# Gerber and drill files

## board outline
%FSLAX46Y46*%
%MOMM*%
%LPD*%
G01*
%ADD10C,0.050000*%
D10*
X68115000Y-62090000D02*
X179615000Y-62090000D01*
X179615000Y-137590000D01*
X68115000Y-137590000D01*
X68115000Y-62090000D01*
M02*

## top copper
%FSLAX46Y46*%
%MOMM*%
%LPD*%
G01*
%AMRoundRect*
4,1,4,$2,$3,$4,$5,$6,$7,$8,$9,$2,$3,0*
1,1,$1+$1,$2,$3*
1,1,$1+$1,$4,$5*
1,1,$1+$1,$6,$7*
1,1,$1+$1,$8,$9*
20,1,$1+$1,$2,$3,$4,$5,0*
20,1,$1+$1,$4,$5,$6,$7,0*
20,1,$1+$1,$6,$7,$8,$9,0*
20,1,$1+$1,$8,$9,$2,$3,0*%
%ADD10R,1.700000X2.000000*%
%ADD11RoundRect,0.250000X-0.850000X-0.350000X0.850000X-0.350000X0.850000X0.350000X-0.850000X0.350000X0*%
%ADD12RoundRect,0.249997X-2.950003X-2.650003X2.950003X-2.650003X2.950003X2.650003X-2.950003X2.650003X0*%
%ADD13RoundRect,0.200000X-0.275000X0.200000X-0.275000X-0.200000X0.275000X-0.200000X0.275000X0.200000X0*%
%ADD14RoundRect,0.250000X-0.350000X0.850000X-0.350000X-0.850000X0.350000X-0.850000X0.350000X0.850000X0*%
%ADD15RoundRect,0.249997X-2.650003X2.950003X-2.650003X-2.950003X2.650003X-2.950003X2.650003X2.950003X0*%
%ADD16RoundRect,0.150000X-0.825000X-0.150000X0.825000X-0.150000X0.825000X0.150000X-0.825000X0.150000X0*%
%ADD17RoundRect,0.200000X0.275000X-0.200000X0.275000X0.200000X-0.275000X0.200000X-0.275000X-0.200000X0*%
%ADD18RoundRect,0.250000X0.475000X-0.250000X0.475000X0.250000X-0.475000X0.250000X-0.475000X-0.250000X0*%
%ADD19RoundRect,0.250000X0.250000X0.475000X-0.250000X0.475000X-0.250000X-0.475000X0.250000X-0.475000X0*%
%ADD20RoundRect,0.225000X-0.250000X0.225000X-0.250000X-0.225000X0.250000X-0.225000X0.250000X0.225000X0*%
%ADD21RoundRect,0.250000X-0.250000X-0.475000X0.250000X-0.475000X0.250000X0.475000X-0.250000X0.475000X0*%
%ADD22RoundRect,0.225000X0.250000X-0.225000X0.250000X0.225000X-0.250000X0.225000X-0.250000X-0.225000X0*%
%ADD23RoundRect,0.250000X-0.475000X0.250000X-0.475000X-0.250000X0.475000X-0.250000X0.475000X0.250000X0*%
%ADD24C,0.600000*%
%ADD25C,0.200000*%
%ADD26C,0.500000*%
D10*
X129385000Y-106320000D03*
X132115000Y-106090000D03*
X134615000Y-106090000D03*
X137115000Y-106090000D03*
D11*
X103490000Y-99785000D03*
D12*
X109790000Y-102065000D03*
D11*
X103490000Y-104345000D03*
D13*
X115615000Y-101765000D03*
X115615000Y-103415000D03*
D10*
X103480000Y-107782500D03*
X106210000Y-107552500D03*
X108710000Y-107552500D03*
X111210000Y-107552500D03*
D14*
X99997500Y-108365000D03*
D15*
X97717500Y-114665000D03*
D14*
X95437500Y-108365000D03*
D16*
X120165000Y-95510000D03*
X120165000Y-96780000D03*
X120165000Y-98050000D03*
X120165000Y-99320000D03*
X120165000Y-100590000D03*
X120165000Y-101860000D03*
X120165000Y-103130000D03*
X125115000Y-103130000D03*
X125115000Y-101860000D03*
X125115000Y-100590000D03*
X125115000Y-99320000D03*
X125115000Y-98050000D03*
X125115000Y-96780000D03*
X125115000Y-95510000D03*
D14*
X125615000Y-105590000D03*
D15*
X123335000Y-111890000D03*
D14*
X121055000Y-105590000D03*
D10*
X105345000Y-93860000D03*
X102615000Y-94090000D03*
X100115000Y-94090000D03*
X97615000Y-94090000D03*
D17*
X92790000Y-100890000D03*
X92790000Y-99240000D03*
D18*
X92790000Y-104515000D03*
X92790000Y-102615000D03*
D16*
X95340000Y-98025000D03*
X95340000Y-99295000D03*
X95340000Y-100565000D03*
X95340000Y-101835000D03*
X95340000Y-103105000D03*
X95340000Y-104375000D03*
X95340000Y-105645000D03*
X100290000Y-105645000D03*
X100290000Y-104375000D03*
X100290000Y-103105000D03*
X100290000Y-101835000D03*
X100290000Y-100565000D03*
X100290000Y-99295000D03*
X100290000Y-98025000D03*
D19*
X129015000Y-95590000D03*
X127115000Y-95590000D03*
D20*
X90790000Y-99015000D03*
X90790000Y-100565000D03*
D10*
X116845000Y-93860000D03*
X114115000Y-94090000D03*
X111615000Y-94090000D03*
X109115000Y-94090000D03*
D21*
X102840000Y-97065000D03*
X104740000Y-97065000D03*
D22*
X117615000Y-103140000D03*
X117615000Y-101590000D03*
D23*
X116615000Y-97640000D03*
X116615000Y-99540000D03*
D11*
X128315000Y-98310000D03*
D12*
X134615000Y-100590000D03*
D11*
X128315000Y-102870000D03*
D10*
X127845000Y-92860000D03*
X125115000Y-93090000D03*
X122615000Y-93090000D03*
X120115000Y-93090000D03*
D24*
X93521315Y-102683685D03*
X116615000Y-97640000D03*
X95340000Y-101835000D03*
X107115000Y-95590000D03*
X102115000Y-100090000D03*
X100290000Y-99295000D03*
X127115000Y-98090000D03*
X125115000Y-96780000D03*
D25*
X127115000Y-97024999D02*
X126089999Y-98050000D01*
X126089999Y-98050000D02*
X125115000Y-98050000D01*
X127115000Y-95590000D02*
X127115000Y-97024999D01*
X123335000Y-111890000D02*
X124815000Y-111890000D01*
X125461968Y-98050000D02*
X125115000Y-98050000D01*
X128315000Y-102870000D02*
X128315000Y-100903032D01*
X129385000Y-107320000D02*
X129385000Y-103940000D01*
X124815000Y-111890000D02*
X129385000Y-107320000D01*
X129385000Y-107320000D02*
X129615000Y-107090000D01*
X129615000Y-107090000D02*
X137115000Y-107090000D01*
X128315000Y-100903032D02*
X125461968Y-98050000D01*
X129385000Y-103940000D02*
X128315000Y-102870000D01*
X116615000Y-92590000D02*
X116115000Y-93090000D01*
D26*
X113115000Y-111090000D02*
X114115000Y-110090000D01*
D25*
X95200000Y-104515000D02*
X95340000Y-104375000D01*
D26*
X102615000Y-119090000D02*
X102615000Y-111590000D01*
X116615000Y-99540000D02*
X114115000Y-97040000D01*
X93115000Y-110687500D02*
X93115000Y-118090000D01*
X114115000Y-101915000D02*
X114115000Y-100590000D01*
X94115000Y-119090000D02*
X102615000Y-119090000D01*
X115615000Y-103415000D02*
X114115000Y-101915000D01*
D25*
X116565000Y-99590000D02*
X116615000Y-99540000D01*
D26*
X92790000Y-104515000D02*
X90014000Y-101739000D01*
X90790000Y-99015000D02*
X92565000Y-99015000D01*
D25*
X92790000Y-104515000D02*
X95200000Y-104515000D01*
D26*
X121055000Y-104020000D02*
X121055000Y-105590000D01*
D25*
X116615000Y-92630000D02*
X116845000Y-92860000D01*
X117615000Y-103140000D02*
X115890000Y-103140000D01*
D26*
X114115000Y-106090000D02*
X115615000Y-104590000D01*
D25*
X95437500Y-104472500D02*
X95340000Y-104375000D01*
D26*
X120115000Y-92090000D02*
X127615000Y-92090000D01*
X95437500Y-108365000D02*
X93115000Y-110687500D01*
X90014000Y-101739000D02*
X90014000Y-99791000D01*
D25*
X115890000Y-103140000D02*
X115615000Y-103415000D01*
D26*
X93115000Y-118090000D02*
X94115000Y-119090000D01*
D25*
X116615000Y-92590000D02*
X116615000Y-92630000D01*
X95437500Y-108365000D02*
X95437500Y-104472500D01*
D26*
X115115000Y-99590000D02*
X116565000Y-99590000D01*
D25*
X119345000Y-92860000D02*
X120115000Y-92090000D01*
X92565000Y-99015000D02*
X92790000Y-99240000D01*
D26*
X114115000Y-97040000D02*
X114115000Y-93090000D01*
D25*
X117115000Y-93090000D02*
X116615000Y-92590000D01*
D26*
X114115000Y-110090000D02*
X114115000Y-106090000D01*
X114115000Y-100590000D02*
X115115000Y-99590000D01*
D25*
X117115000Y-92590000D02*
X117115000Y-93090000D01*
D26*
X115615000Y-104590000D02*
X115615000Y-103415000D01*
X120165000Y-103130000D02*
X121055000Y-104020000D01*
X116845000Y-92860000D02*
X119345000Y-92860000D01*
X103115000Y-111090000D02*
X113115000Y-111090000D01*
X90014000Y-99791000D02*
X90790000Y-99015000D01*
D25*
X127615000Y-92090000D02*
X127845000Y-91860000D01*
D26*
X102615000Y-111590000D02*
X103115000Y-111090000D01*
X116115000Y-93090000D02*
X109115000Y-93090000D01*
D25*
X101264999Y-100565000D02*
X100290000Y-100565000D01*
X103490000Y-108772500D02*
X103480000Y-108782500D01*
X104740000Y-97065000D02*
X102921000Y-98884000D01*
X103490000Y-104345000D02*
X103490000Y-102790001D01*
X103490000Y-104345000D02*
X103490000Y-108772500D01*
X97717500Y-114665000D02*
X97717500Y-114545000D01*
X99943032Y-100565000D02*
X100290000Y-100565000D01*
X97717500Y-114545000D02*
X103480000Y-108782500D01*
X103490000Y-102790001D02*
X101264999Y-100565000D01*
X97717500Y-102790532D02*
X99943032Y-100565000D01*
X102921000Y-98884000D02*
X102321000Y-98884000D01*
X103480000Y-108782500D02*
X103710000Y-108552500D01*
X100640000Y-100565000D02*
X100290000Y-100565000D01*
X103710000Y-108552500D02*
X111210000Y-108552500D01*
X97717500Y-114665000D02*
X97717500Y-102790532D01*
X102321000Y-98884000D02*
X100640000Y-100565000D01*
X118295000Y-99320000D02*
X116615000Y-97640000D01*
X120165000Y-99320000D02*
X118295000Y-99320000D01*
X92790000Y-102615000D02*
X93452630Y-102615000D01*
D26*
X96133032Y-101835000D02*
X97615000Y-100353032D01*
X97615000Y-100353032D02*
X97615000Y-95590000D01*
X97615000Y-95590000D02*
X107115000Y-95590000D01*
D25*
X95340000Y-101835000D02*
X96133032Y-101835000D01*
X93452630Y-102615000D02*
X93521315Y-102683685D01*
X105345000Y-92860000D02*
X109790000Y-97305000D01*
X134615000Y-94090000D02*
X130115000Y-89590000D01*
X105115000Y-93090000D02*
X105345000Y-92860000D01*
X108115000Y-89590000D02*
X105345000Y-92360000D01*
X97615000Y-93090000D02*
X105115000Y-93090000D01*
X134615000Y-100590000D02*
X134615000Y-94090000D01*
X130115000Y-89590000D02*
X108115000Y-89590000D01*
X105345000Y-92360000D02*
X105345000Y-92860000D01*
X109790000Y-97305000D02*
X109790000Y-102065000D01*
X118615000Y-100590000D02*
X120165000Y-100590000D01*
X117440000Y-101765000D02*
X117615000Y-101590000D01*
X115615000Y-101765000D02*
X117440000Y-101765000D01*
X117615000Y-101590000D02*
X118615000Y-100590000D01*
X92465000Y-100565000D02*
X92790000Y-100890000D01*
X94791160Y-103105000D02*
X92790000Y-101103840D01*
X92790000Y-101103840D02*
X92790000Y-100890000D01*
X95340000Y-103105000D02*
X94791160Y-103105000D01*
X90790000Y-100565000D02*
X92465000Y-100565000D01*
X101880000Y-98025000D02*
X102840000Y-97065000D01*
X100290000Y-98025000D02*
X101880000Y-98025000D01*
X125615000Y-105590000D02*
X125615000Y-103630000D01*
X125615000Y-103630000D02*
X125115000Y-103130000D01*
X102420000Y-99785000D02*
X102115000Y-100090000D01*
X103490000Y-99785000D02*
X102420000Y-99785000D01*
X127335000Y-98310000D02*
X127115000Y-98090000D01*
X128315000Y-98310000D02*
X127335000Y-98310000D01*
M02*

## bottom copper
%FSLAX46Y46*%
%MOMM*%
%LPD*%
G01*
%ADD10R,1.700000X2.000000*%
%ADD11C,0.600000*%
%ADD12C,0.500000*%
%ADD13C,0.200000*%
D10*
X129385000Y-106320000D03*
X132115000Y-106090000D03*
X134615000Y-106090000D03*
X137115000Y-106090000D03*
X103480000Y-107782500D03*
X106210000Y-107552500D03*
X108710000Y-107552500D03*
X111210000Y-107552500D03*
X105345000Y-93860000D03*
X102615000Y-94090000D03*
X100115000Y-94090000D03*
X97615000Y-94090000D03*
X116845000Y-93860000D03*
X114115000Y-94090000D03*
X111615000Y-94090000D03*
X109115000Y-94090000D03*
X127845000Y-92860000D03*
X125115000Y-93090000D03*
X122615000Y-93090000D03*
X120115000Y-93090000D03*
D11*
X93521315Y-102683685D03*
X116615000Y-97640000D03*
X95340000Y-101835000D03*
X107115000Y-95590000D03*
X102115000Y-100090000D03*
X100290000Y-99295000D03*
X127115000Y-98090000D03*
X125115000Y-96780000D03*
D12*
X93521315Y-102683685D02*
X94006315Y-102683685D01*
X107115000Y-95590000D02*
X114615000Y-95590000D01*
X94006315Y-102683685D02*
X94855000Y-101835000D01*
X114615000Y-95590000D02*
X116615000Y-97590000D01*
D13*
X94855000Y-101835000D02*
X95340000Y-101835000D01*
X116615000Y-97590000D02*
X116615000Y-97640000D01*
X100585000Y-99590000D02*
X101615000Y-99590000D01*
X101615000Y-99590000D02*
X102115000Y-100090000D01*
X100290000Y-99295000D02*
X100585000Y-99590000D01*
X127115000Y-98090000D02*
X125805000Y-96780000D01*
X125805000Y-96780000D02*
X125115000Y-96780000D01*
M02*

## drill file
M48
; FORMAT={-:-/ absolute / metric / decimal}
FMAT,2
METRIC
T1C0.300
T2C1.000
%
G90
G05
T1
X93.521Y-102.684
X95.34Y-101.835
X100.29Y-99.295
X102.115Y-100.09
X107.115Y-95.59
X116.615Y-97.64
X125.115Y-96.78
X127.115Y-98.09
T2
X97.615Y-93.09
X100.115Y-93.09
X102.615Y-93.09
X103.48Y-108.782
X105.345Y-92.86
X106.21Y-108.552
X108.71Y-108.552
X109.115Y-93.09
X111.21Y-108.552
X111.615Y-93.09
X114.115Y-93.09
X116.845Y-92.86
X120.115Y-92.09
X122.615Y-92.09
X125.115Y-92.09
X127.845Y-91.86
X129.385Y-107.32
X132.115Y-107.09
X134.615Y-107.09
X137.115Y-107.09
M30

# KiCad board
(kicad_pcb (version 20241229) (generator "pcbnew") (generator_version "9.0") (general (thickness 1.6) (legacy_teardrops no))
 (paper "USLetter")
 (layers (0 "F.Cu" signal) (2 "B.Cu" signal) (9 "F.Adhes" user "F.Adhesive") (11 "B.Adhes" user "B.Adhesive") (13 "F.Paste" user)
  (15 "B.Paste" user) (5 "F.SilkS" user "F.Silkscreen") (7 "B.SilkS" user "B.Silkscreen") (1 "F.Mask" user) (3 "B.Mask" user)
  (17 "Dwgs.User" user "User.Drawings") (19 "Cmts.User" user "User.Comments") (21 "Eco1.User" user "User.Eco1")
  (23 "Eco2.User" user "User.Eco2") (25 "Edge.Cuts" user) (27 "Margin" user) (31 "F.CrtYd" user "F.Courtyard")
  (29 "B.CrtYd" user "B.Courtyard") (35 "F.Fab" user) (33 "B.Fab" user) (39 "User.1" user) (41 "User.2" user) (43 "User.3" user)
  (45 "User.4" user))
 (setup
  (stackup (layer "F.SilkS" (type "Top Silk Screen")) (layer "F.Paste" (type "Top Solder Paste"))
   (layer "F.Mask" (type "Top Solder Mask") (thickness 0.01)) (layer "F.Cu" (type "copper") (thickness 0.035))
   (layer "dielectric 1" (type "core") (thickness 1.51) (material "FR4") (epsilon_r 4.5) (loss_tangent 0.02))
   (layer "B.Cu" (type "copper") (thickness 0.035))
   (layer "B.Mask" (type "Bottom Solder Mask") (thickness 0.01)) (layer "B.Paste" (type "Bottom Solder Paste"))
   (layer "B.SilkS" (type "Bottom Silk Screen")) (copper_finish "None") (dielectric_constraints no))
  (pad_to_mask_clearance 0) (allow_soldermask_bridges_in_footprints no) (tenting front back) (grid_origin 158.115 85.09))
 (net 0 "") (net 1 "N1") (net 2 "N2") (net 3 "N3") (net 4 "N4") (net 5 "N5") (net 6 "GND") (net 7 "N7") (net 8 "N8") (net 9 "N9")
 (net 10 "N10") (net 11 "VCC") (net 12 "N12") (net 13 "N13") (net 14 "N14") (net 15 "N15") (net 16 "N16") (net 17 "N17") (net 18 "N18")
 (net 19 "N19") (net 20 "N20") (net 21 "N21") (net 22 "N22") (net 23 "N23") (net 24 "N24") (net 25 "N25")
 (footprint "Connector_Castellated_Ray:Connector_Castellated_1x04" (layer "F.Cu") (at 132.115 106.09 90)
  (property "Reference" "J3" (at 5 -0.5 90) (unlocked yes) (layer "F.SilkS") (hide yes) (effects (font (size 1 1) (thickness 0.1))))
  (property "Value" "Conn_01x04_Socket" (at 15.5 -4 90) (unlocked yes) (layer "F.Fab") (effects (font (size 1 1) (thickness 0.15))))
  (pad "1" thru_hole rect (at -1.23 -2.73 90) (size 2 1.7) (drill 1 (offset 1 0)) (layers "*.Cu" "*.Mask") (remove_unused_layers no)
   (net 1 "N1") (solder_mask_margin 0.04))
  (pad "2" thru_hole rect (at -1 0 90) (size 2 1.7) (drill 1 (offset 1 0)) (layers "*.Cu" "*.Mask") (remove_unused_layers no) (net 1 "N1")
   (solder_mask_margin 0.04))
  (pad "3" thru_hole rect (at -1 2.5 90) (size 2 1.7) (drill 1 (offset 1 0)) (layers "*.Cu" "*.Mask") (remove_unused_layers no) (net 1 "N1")
   (solder_mask_margin 0.04))
  (pad "4" thru_hole rect (at -1 5 90) (size 2 1.7) (drill 1 (offset 1 0)) (layers "*.Cu" "*.Mask") (remove_unused_layers no) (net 1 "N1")
   (solder_mask_margin 0.04)))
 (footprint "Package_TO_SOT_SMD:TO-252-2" (layer "F.Cu") (at 108.53 102.065)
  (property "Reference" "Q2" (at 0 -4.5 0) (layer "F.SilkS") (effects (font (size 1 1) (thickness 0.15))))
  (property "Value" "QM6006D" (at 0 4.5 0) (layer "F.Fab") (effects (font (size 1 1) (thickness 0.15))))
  (pad "" smd roundrect (at -0.415 -1.525) (size 3.05 2.75) (layers "F.Paste") (roundrect_rratio 0.090909))
  (pad "" smd roundrect (at -0.415 1.525) (size 3.05 2.75) (layers "F.Paste") (roundrect_rratio 0.090909))
  (pad "" smd roundrect (at 2.935 -1.525) (size 3.05 2.75) (layers "F.Paste") (roundrect_rratio 0.090909))
  (pad "" smd roundrect (at 2.935 1.525) (size 3.05 2.75) (layers "F.Paste") (roundrect_rratio 0.090909))
  (pad "1" smd roundrect (at -5.04 -2.28) (size 2.2 1.2) (layers "F.Cu" "F.Mask" "F.Paste") (roundrect_rratio 0.208333) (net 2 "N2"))
  (pad "2" smd roundrect (at 1.26 0) (size 6.4 5.8) (layers "F.Cu" "F.Mask") (roundrect_rratio 0.043103) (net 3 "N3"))
  (pad "3" smd roundrect (at -5.04 2.28) (size 2.2 1.2) (layers "F.Cu" "F.Mask" "F.Paste") (roundrect_rratio 0.208333) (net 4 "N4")))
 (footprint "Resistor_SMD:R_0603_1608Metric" (layer "F.Cu") (at 115.615 102.59 -90)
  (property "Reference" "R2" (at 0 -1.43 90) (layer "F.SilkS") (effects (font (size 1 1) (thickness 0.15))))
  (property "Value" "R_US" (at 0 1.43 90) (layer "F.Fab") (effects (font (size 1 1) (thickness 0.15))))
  (pad "1" smd roundrect (at -0.825 0 270) (size 0.8 0.95) (layers "F.Cu" "F.Mask" "F.Paste") (roundrect_rratio 0.25) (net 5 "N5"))
  (pad "2" smd roundrect (at 0.825 0 270) (size 0.8 0.95) (layers "F.Cu" "F.Mask" "F.Paste") (roundrect_rratio 0.25) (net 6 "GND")))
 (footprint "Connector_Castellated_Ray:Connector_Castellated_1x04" (layer "F.Cu") (at 106.21 107.5525 90)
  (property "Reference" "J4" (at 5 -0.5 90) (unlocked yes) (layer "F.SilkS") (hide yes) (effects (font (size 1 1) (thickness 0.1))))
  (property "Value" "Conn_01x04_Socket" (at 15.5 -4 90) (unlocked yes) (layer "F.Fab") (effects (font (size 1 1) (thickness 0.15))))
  (pad "1" thru_hole rect (at -1.23 -2.73 90) (size 2 1.7) (drill 1 (offset 1 0)) (layers "*.Cu" "*.Mask") (remove_unused_layers no)
   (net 4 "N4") (solder_mask_margin 0.04))
  (pad "2" thru_hole rect (at -1 0 90) (size 2 1.7) (drill 1 (offset 1 0)) (layers "*.Cu" "*.Mask") (remove_unused_layers no) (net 4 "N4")
   (solder_mask_margin 0.04))
  (pad "3" thru_hole rect (at -1 2.5 90) (size 2 1.7) (drill 1 (offset 1 0)) (layers "*.Cu" "*.Mask") (remove_unused_layers no) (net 4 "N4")
   (solder_mask_margin 0.04))
  (pad "4" thru_hole rect (at -1 5 90) (size 2 1.7) (drill 1 (offset 1 0)) (layers "*.Cu" "*.Mask") (remove_unused_layers no) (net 4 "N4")
   (solder_mask_margin 0.04)))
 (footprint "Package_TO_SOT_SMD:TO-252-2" (layer "F.Cu") (at 97.7175 113.405 -90)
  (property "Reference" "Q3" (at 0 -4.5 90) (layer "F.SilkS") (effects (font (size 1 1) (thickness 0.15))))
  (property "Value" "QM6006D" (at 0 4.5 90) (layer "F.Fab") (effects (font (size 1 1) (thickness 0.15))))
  (pad "" smd roundrect (at -0.415 -1.525 270) (size 3.05 2.75) (layers "F.Paste") (roundrect_rratio 0.090909))
  (pad "" smd roundrect (at -0.415 1.525 270) (size 3.05 2.75) (layers "F.Paste") (roundrect_rratio 0.090909))
  (pad "" smd roundrect (at 2.935 -1.525 270) (size 3.05 2.75) (layers "F.Paste") (roundrect_rratio 0.090909))
  (pad "" smd roundrect (at 2.935 1.525 270) (size 3.05 2.75) (layers "F.Paste") (roundrect_rratio 0.090909))
  (pad "1" smd roundrect (at -5.04 -2.28 270) (size 2.2 1.2) (layers "F.Cu" "F.Mask" "F.Paste") (roundrect_rratio 0.208333) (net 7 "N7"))
  (pad "2" smd roundrect (at 1.26 0 270) (size 6.4 5.8) (layers "F.Cu" "F.Mask") (roundrect_rratio 0.043103) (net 4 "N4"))
  (pad "3" smd roundrect (at -5.04 2.28 270) (size 2.2 1.2) (layers "F.Cu" "F.Mask" "F.Paste") (roundrect_rratio 0.208333) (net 6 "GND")))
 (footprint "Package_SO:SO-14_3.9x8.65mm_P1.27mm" (layer "F.Cu") (at 122.64 99.32)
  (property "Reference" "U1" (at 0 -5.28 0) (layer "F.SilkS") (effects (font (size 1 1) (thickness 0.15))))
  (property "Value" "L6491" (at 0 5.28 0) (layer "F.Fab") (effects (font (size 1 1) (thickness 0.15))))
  (pad "1" smd roundrect (at -2.475 -3.81) (size 1.95 0.6) (layers "F.Cu" "F.Mask" "F.Paste") (roundrect_rratio 0.25) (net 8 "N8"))
  (pad "2" smd roundrect (at -2.475 -2.54) (size 1.95 0.6) (layers "F.Cu" "F.Mask" "F.Paste") (roundrect_rratio 0.25) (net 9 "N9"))
  (pad "3" smd roundrect (at -2.475 -1.27) (size 1.95 0.6) (layers "F.Cu" "F.Mask" "F.Paste") (roundrect_rratio 0.25) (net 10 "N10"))
  (pad "4" smd roundrect (at -2.475 0) (size 1.95 0.6) (layers "F.Cu" "F.Mask" "F.Paste") (roundrect_rratio 0.25) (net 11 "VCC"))
  (pad "5" smd roundrect (at -2.475 1.27) (size 1.95 0.6) (layers "F.Cu" "F.Mask" "F.Paste") (roundrect_rratio 0.25) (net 5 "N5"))
  (pad "6" smd roundrect (at -2.475 2.54) (size 1.95 0.6) (layers "F.Cu" "F.Mask" "F.Paste") (roundrect_rratio 0.25) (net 6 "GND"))
  (pad "7" smd roundrect (at -2.475 3.81) (size 1.95 0.6) (layers "F.Cu" "F.Mask" "F.Paste") (roundrect_rratio 0.25) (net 6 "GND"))
  (pad "8" smd roundrect (at 2.475 3.81) (size 1.95 0.6) (layers "F.Cu" "F.Mask" "F.Paste") (roundrect_rratio 0.25) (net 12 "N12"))
  (pad "9" smd roundrect (at 2.475 2.54) (size 1.95 0.6) (layers "F.Cu" "F.Mask" "F.Paste") (roundrect_rratio 0.25) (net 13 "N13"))
  (pad "10" smd roundrect (at 2.475 1.27) (size 1.95 0.6) (layers "F.Cu" "F.Mask" "F.Paste") (roundrect_rratio 0.25) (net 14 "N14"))
  (pad "11" smd roundrect (at 2.475 0) (size 1.95 0.6) (layers "F.Cu" "F.Mask" "F.Paste") (roundrect_rratio 0.25) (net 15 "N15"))
  (pad "12" smd roundrect (at 2.475 -1.27) (size 1.95 0.6) (layers "F.Cu" "F.Mask" "F.Paste") (roundrect_rratio 0.25) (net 1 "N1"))
  (pad "13" smd roundrect (at 2.475 -2.54) (size 1.95 0.6) (layers "F.Cu" "F.Mask" "F.Paste") (roundrect_rratio 0.25) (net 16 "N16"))
  (pad "14" smd roundrect (at 2.475 -3.81) (size 1.95 0.6) (layers "F.Cu" "F.Mask" "F.Paste") (roundrect_rratio 0.25) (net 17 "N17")))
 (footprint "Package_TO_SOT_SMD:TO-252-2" (layer "F.Cu") (at 123.335 110.63 -90)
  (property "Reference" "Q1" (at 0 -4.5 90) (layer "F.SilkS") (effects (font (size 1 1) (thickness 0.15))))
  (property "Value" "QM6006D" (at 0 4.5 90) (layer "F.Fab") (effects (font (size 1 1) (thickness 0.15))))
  (pad "" smd roundrect (at -0.415 -1.525 270) (size 3.05 2.75) (layers "F.Paste") (roundrect_rratio 0.090909))
  (pad "" smd roundrect (at -0.415 1.525 270) (size 3.05 2.75) (layers "F.Paste") (roundrect_rratio 0.090909))
  (pad "" smd roundrect (at 2.935 -1.525 270) (size 3.05 2.75) (layers "F.Paste") (roundrect_rratio 0.090909))
  (pad "" smd roundrect (at 2.935 1.525 270) (size 3.05 2.75) (layers "F.Paste") (roundrect_rratio 0.090909))
  (pad "1" smd roundrect (at -5.04 -2.28 270) (size 2.2 1.2) (layers "F.Cu" "F.Mask" "F.Paste") (roundrect_rratio 0.208333) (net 12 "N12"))
  (pad "2" smd roundrect (at 1.26 0 270) (size 6.4 5.8) (layers "F.Cu" "F.Mask") (roundrect_rratio 0.043103) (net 1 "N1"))
  (pad "3" smd roundrect (at -5.04 2.28 270) (size 2.2 1.2) (layers "F.Cu" "F.Mask" "F.Paste") (roundrect_rratio 0.208333) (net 6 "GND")))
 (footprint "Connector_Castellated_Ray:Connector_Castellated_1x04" (layer "F.Cu") (at 102.615 94.09 -90)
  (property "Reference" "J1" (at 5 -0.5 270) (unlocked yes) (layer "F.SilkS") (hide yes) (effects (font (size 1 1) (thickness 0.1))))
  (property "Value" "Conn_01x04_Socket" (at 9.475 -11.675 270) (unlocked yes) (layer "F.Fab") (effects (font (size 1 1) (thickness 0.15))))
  (pad "1" thru_hole rect (at -1.23 -2.73 270) (size 2 1.7) (drill 1 (offset 1 0)) (layers "*.Cu" "*.Mask") (remove_unused_layers no)
   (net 3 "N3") (solder_mask_margin 0.04))
  (pad "2" thru_hole rect (at -1 0 270) (size 2 1.7) (drill 1 (offset 1 0)) (layers "*.Cu" "*.Mask") (remove_unused_layers no) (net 3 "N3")
   (solder_mask_margin 0.04))
  (pad "3" thru_hole rect (at -1 2.5 270) (size 2 1.7) (drill 1 (offset 1 0)) (layers "*.Cu" "*.Mask") (remove_unused_layers no)
   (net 3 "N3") (solder_mask_margin 0.04))
  (pad "4" thru_hole rect (at -1 5 270) (size 2 1.7) (drill 1 (offset 1 0)) (layers "*.Cu" "*.Mask") (remove_unused_layers no) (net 3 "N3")
   (solder_mask_margin 0.04)))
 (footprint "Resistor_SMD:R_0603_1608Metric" (layer "F.Cu") (at 92.79 100.065 90)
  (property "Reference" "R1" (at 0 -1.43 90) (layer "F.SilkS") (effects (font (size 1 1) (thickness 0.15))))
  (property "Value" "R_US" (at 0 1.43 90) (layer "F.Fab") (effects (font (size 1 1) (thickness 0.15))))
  (pad "1" smd roundrect (at -0.825 0 90) (size 0.8 0.95) (layers "F.Cu" "F.Mask" "F.Paste") (roundrect_rratio 0.25) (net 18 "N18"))
  (pad "2" smd roundrect (at 0.825 0 90) (size 0.8 0.95) (layers "F.Cu" "F.Mask" "F.Paste") (roundrect_rratio 0.25) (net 6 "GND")))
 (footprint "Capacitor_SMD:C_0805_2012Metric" (layer "F.Cu") (at 92.79 103.565 90)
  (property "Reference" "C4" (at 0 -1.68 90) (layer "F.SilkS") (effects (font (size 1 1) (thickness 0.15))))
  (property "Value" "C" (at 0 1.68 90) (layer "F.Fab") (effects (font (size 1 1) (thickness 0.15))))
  (pad "1" smd roundrect (at -0.95 0 90) (size 1 1.45) (layers "F.Cu" "F.Mask" "F.Paste") (roundrect_rratio 0.25) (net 6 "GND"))
  (pad "2" smd roundrect (at 0.95 0 90) (size 1 1.45) (layers "F.Cu" "F.Mask" "F.Paste") (roundrect_rratio 0.25) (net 11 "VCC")))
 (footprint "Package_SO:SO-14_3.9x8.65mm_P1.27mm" (layer "F.Cu") (at 97.815 101.835)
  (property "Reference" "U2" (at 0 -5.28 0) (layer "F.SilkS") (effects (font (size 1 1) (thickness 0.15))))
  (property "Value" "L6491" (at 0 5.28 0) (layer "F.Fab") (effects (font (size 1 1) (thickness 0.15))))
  (pad "1" smd roundrect (at -2.475 -3.81) (size 1.95 0.6) (layers "F.Cu" "F.Mask" "F.Paste") (roundrect_rratio 0.25) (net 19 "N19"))
  (pad "2" smd roundrect (at -2.475 -2.54) (size 1.95 0.6) (layers "F.Cu" "F.Mask" "F.Paste") (roundrect_rratio 0.25) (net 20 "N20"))
  (pad "3" smd roundrect (at -2.475 -1.27) (size 1.95 0.6) (layers "F.Cu" "F.Mask" "F.Paste") (roundrect_rratio 0.25) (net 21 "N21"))
  (pad "4" smd roundrect (at -2.475 0) (size 1.95 0.6) (layers "F.Cu" "F.Mask" "F.Paste") (roundrect_rratio 0.25) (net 11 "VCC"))
  (pad "5" smd roundrect (at -2.475 1.27) (size 1.95 0.6) (layers "F.Cu" "F.Mask" "F.Paste") (roundrect_rratio 0.25) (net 18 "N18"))
  (pad "6" smd roundrect (at -2.475 2.54) (size 1.95 0.6) (layers "F.Cu" "F.Mask" "F.Paste") (roundrect_rratio 0.25) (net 6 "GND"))
  (pad "7" smd roundrect (at -2.475 3.81) (size 1.95 0.6) (layers "F.Cu" "F.Mask" "F.Paste") (roundrect_rratio 0.25) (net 6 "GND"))
  (pad "8" smd roundrect (at 2.475 3.81) (size 1.95 0.6) (layers "F.Cu" "F.Mask" "F.Paste") (roundrect_rratio 0.25) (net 7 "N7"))
  (pad "9" smd roundrect (at 2.475 2.54) (size 1.95 0.6) (layers "F.Cu" "F.Mask" "F.Paste") (roundrect_rratio 0.25) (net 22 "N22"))
  (pad "10" smd roundrect (at 2.475 1.27) (size 1.95 0.6) (layers "F.Cu" "F.Mask" "F.Paste") (roundrect_rratio 0.25) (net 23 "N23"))
  (pad "11" smd roundrect (at 2.475 0) (size 1.95 0.6) (layers "F.Cu" "F.Mask" "F.Paste") (roundrect_rratio 0.25) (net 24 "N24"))
  (pad "12" smd roundrect (at 2.475 -1.27) (size 1.95 0.6) (layers "F.Cu" "F.Mask" "F.Paste") (roundrect_rratio 0.25) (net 4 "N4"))
  (pad "13" smd roundrect (at 2.475 -2.54) (size 1.95 0.6) (layers "F.Cu" "F.Mask" "F.Paste") (roundrect_rratio 0.25) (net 2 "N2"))
  (pad "14" smd roundrect (at 2.475 -3.81) (size 1.95 0.6) (layers "F.Cu" "F.Mask" "F.Paste") (roundrect_rratio 0.25) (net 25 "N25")))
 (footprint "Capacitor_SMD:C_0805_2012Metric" (layer "F.Cu") (at 128.065 95.59 180)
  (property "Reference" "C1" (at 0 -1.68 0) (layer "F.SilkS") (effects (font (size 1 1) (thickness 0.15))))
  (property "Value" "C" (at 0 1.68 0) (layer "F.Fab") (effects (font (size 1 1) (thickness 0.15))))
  (pad "1" smd roundrect (at -0.95 0 180) (size 1 1.45) (layers "F.Cu" "F.Mask" "F.Paste") (roundrect_rratio 0.25) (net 17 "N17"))
  (pad "2" smd roundrect (at 0.95 0 180) (size 1 1.45) (layers "F.Cu" "F.Mask" "F.Paste") (roundrect_rratio 0.25) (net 1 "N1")))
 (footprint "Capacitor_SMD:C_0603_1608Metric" (layer "F.Cu") (at 90.79 99.79 -90)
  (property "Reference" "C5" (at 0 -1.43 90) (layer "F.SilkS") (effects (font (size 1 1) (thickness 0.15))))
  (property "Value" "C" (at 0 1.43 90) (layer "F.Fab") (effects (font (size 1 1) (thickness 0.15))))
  (pad "1" smd roundrect (at -0.775 0 270) (size 0.9 0.95) (layers "F.Cu" "F.Mask" "F.Paste") (roundrect_rratio 0.25) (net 6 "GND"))
  (pad "2" smd roundrect (at 0.775 0 270) (size 0.9 0.95) (layers "F.Cu" "F.Mask" "F.Paste") (roundrect_rratio 0.25) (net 18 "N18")))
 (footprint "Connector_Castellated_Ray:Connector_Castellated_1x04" (layer "F.Cu") (at 114.115 94.09 -90)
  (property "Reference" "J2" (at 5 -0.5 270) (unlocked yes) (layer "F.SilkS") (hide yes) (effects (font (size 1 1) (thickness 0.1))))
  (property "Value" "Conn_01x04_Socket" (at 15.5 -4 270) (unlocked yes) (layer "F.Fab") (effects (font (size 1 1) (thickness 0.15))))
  (pad "1" thru_hole rect (at -1.23 -2.73 270) (size 2 1.7) (drill 1 (offset 1 0)) (layers "*.Cu" "*.Mask") (remove_unused_layers no)
   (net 6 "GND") (solder_mask_margin 0.04))
  (pad "2" thru_hole rect (at -1 0 270) (size 2 1.7) (drill 1 (offset 1 0)) (layers "*.Cu" "*.Mask") (remove_unused_layers no) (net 6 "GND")
   (solder_mask_margin 0.04))
  (pad "3" thru_hole rect (at -1 2.5 270) (size 2 1.7) (drill 1 (offset 1 0)) (layers "*.Cu" "*.Mask") (remove_unused_layers no)
   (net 6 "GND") (solder_mask_margin 0.04))
  (pad "4" thru_hole rect (at -1 5 270) (size 2 1.7) (drill 1 (offset 1 0)) (layers "*.Cu" "*.Mask") (remove_unused_layers no) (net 6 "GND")
   (solder_mask_margin 0.04)))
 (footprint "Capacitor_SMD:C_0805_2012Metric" (layer "F.Cu") (at 103.79 97.065)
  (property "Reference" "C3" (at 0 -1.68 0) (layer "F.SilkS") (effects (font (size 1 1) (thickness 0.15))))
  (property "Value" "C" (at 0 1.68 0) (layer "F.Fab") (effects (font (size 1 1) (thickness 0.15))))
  (pad "1" smd roundrect (at -0.95 0) (size 1 1.45) (layers "F.Cu" "F.Mask" "F.Paste") (roundrect_rratio 0.25) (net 25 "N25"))
  (pad "2" smd roundrect (at 0.95 0) (size 1 1.45) (layers "F.Cu" "F.Mask" "F.Paste") (roundrect_rratio 0.25) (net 4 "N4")))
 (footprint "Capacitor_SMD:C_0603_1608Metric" (layer "F.Cu") (at 117.615 102.365 90)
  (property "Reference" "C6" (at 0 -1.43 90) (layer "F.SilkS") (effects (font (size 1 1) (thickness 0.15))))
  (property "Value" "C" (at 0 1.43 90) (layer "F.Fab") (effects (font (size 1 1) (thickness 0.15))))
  (pad "1" smd roundrect (at -0.775 0 90) (size 0.9 0.95) (layers "F.Cu" "F.Mask" "F.Paste") (roundrect_rratio 0.25) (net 6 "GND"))
  (pad "2" smd roundrect (at 0.775 0 90) (size 0.9 0.95) (layers "F.Cu" "F.Mask" "F.Paste") (roundrect_rratio 0.25) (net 5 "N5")))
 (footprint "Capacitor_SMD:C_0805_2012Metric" (layer "F.Cu") (at 116.615 98.59 -90)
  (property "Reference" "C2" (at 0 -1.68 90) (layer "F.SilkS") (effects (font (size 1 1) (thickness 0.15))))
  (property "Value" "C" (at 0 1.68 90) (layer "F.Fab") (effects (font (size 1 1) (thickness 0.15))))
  (pad "1" smd roundrect (at -0.95 0 270) (size 1 1.45) (layers "F.Cu" "F.Mask" "F.Paste") (roundrect_rratio 0.25) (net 11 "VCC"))
  (pad "2" smd roundrect (at 0.95 0 270) (size 1 1.45) (layers "F.Cu" "F.Mask" "F.Paste") (roundrect_rratio 0.25) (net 6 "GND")))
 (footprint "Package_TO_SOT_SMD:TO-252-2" (layer "F.Cu") (at 133.355 100.59)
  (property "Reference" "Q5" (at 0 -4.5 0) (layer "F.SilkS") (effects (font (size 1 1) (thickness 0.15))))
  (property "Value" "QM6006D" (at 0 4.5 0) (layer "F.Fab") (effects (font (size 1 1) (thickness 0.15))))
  (pad "" smd roundrect (at -0.415 -1.525) (size 3.05 2.75) (layers "F.Paste") (roundrect_rratio 0.090909))
  (pad "" smd roundrect (at -0.415 1.525) (size 3.05 2.75) (layers "F.Paste") (roundrect_rratio 0.090909))
  (pad "" smd roundrect (at 2.935 -1.525) (size 3.05 2.75) (layers "F.Paste") (roundrect_rratio 0.090909))
  (pad "" smd roundrect (at 2.935 1.525) (size 3.05 2.75) (layers "F.Paste") (roundrect_rratio 0.090909))
  (pad "1" smd roundrect (at -5.04 -2.28) (size 2.2 1.2) (layers "F.Cu" "F.Mask" "F.Paste") (roundrect_rratio 0.208333) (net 16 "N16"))
  (pad "2" smd roundrect (at 1.26 0) (size 6.4 5.8) (layers "F.Cu" "F.Mask") (roundrect_rratio 0.043103) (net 3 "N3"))
  (pad "3" smd roundrect (at -5.04 2.28) (size 2.2 1.2) (layers "F.Cu" "F.Mask" "F.Paste") (roundrect_rratio 0.208333) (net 1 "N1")))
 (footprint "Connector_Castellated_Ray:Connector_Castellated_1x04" (layer "F.Cu") (at 125.115 93.09 -90)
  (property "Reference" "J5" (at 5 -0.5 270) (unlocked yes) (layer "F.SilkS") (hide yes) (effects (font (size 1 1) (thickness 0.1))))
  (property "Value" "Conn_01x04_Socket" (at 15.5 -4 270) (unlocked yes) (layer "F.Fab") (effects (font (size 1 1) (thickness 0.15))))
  (pad "1" thru_hole rect (at -1.23 -2.73 270) (size 2 1.7) (drill 1 (offset 1 0)) (layers "*.Cu" "*.Mask") (remove_unused_layers no)
   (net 6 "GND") (solder_mask_margin 0.04))
  (pad "2" thru_hole rect (at -1 0 270) (size 2 1.7) (drill 1 (offset 1 0)) (layers "*.Cu" "*.Mask") (remove_unused_layers no) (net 6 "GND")
   (solder_mask_margin 0.04))
  (pad "3" thru_hole rect (at -1 2.5 270) (size 2 1.7) (drill 1 (offset 1 0)) (layers "*.Cu" "*.Mask") (remove_unused_layers no)
   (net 6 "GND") (solder_mask_margin 0.04))
  (pad "4" thru_hole rect (at -1 5 270) (size 2 1.7) (drill 1 (offset 1 0)) (layers "*.Cu" "*.Mask") (remove_unused_layers no) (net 6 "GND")
   (solder_mask_margin 0.04)))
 (gr_rect (start 68.115 62.09) (end 179.615 137.59) (stroke (width 0.05) (type default)) (fill no) (layer "Edge.Cuts"))
 (segment (start 127.115 97.024999) (end 126.089999 98.05) (width 0.2) (layer "F.Cu") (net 1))
 (segment (start 126.089999 98.05) (end 125.115 98.05) (width 0.2) (layer "F.Cu") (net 1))
 (segment (start 127.115 95.59) (end 127.115 97.024999) (width 0.2) (layer "F.Cu") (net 1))
 (segment (start 123.335 111.89) (end 124.815 111.89) (width 0.2) (layer "F.Cu") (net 1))
 (segment (start 125.461968 98.05) (end 125.115 98.05) (width 0.2) (layer "F.Cu") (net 1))
 (segment (start 128.315 102.87) (end 128.315 100.903032) (width 0.2) (layer "F.Cu") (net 1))
 (segment (start 129.385 107.32) (end 129.385 103.94) (width 0.2) (layer "F.Cu") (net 1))
 (segment (start 124.815 111.89) (end 129.385 107.32) (width 0.2) (layer "F.Cu") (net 1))
 (segment (start 129.385 107.32) (end 129.615 107.09) (width 0.2) (layer "F.Cu") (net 1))
 (segment (start 129.615 107.09) (end 137.115 107.09) (width 0.2) (layer "F.Cu") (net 1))
 (segment (start 128.315 100.903032) (end 125.461968 98.05) (width 0.2) (layer "F.Cu") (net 1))
 (segment (start 129.385 103.94) (end 128.315 102.87) (width 0.2) (layer "F.Cu") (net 1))
 (segment (start 116.615 92.59) (end 116.115 93.09) (width 0.2) (layer "F.Cu") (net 6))
 (segment (start 113.115 111.09) (end 114.115 110.09) (width 0.5) (layer "F.Cu") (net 6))
 (segment (start 95.2 104.515) (end 95.34 104.375) (width 0.2) (layer "F.Cu") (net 6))
 (segment (start 102.615 119.09) (end 102.615 111.59) (width 0.5) (layer "F.Cu") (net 6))
 (segment (start 116.615 99.54) (end 114.115 97.04) (width 0.5) (layer "F.Cu") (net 6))
 (segment (start 93.115 110.6875) (end 93.115 118.09) (width 0.5) (layer "F.Cu") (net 6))
 (segment (start 114.115 101.915) (end 114.115 100.59) (width 0.5) (layer "F.Cu") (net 6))
 (segment (start 94.115 119.09) (end 102.615 119.09) (width 0.5) (layer "F.Cu") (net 6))
 (segment (start 115.615 103.415) (end 114.115 101.915) (width 0.5) (layer "F.Cu") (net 6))
 (segment (start 116.565 99.59) (end 116.615 99.54) (width 0.2) (layer "F.Cu") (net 6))
 (segment (start 92.79 104.515) (end 90.014 101.739) (width 0.5) (layer "F.Cu") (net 6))
 (segment (start 90.79 99.015) (end 92.565 99.015) (width 0.5) (layer "F.Cu") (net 6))
 (segment (start 92.79 104.515) (end 95.2 104.515) (width 0.2) (layer "F.Cu") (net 6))
 (segment (start 121.055 104.02) (end 121.055 105.59) (width 0.5) (layer "F.Cu") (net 6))
 (segment (start 116.615 92.63) (end 116.845 92.86) (width 0.2) (layer "F.Cu") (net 6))
 (segment (start 117.615 103.14) (end 115.89 103.14) (width 0.2) (layer "F.Cu") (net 6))
 (segment (start 114.115 106.09) (end 115.615 104.59) (width 0.5) (layer "F.Cu") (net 6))
 (segment (start 95.4375 104.4725) (end 95.34 104.375) (width 0.2) (layer "F.Cu") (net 6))
 (segment (start 120.115 92.09) (end 127.615 92.09) (width 0.5) (layer "F.Cu") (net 6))
 (segment (start 95.4375 108.365) (end 93.115 110.6875) (width 0.5) (layer "F.Cu") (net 6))
 (segment (start 90.014 101.739) (end 90.014 99.791) (width 0.5) (layer "F.Cu") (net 6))
 (segment (start 115.89 103.14) (end 115.615 103.415) (width 0.2) (layer "F.Cu") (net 6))
 (segment (start 93.115 118.09) (end 94.115 119.09) (width 0.5) (layer "F.Cu") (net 6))
 (segment (start 116.615 92.59) (end 116.615 92.63) (width 0.2) (layer "F.Cu") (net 6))
 (segment (start 95.4375 108.365) (end 95.4375 104.4725) (width 0.2) (layer "F.Cu") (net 6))
 (segment (start 115.115 99.59) (end 116.565 99.59) (width 0.5) (layer "F.Cu") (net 6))
 (segment (start 119.345 92.86) (end 120.115 92.09) (width 0.2) (layer "F.Cu") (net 6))
 (segment (start 92.565 99.015) (end 92.79 99.24) (width 0.2) (layer "F.Cu") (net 6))
 (segment (start 114.115 97.04) (end 114.115 93.09) (width 0.5) (layer "F.Cu") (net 6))
 (segment (start 117.115 93.09) (end 116.615 92.59) (width 0.2) (layer "F.Cu") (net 6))
 (segment (start 114.115 110.09) (end 114.115 106.09) (width 0.5) (layer "F.Cu") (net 6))
 (segment (start 114.115 100.59) (end 115.115 99.59) (width 0.5) (layer "F.Cu") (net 6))
 (segment (start 117.115 92.59) (end 117.115 93.09) (width 0.2) (layer "F.Cu") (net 6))
 (segment (start 115.615 104.59) (end 115.615 103.415) (width 0.5) (layer "F.Cu") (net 6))
 (segment (start 120.165 103.13) (end 121.055 104.02) (width 0.5) (layer "F.Cu") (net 6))
 (segment (start 116.845 92.86) (end 119.345 92.86) (width 0.5) (layer "F.Cu") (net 6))
 (segment (start 103.115 111.09) (end 113.115 111.09) (width 0.5) (layer "F.Cu") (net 6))
 (segment (start 90.014 99.791) (end 90.79 99.015) (width 0.5) (layer "F.Cu") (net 6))
 (segment (start 127.615 92.09) (end 127.845 91.86) (width 0.2) (layer "F.Cu") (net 6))
 (segment (start 102.615 111.59) (end 103.115 111.09) (width 0.5) (layer "F.Cu") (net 6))
 (segment (start 116.115 93.09) (end 109.115 93.09) (width 0.5) (layer "F.Cu") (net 6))
 (segment (start 101.264999 100.565) (end 100.29 100.565) (width 0.2) (layer "F.Cu") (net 4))
 (segment (start 103.49 108.7725) (end 103.48 108.7825) (width 0.2) (layer "F.Cu") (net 4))
 (segment (start 104.74 97.065) (end 102.921 98.884) (width 0.2) (layer "F.Cu") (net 4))
 (segment (start 103.49 104.345) (end 103.49 102.790001) (width 0.2) (layer "F.Cu") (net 4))
 (segment (start 103.49 104.345) (end 103.49 108.7725) (width 0.2) (layer "F.Cu") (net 4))
 (segment (start 97.7175 114.665) (end 97.7175 114.545) (width 0.2) (layer "F.Cu") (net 4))
 (segment (start 99.943032 100.565) (end 100.29 100.565) (width 0.2) (layer "F.Cu") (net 4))
 (segment (start 97.7175 114.545) (end 103.48 108.7825) (width 0.2) (layer "F.Cu") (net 4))
 (segment (start 103.49 102.790001) (end 101.264999 100.565) (width 0.2) (layer "F.Cu") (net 4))
 (segment (start 97.7175 102.790532) (end 99.943032 100.565) (width 0.2) (layer "F.Cu") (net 4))
 (segment (start 102.921 98.884) (end 102.321 98.884) (width 0.2) (layer "F.Cu") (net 4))
 (segment (start 103.48 108.7825) (end 103.71 108.5525) (width 0.2) (layer "F.Cu") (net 4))
 (segment (start 100.64 100.565) (end 100.29 100.565) (width 0.2) (layer "F.Cu") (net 4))
 (segment (start 103.71 108.5525) (end 111.21 108.5525) (width 0.2) (layer "F.Cu") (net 4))
 (segment (start 97.7175 114.665) (end 97.7175 102.790532) (width 0.2) (layer "F.Cu") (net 4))
 (segment (start 102.321 98.884) (end 100.64 100.565) (width 0.2) (layer "F.Cu") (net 4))
 (segment (start 118.295 99.32) (end 116.615 97.64) (width 0.2) (layer "F.Cu") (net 11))
 (segment (start 120.165 99.32) (end 118.295 99.32) (width 0.2) (layer "F.Cu") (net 11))
 (segment (start 92.79 102.615) (end 93.45263 102.615) (width 0.2) (layer "F.Cu") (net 11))
 (segment (start 96.133032 101.835) (end 97.615 100.353032) (width 0.5) (layer "F.Cu") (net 11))
 (segment (start 97.615 100.353032) (end 97.615 95.59) (width 0.5) (layer "F.Cu") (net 11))
 (segment (start 97.615 95.59) (end 107.115 95.59) (width 0.5) (layer "F.Cu") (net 11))
 (segment (start 95.34 101.835) (end 96.133032 101.835) (width 0.2) (layer "F.Cu") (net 11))
 (segment (start 93.45263 102.615) (end 93.521315 102.683685) (width 0.2) (layer "F.Cu") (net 11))
 (via (at 93.521315 102.683685) (size 0.6) (drill 0.3) (layers "F.Cu" "B.Cu") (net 11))
 (via (at 116.615 97.64) (size 0.6) (drill 0.3) (layers "F.Cu" "B.Cu") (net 11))
 (via (at 95.34 101.835) (size 0.6) (drill 0.3) (layers "F.Cu" "B.Cu") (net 11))
 (via (at 107.115 95.59) (size 0.6) (drill 0.3) (layers "F.Cu" "B.Cu") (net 11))
 (segment (start 93.521315 102.683685) (end 94.006315 102.683685) (width 0.5) (layer "B.Cu") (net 11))
 (segment (start 107.115 95.59) (end 114.615 95.59) (width 0.5) (layer "B.Cu") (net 11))
 (segment (start 94.006315 102.683685) (end 94.855 101.835) (width 0.5) (layer "B.Cu") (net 11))
 (segment (start 114.615 95.59) (end 116.615 97.59) (width 0.5) (layer "B.Cu") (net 11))
 (segment (start 94.855 101.835) (end 95.34 101.835) (width 0.2) (layer "B.Cu") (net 11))
 (segment (start 116.615 97.59) (end 116.615 97.64) (width 0.2) (layer "B.Cu") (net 11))
 (segment (start 105.345 92.86) (end 109.79 97.305) (width 0.2) (layer "F.Cu") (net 3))
 (segment (start 134.615 94.09) (end 130.115 89.59) (width 0.2) (layer "F.Cu") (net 3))
 (segment (start 105.115 93.09) (end 105.345 92.86) (width 0.2) (layer "F.Cu") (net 3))
 (segment (start 108.115 89.59) (end 105.345 92.36) (width 0.2) (layer "F.Cu") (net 3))
 (segment (start 97.615 93.09) (end 105.115 93.09) (width 0.2) (layer "F.Cu") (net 3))
 (segment (start 134.615 100.59) (end 134.615 94.09) (width 0.2) (layer "F.Cu") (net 3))
 (segment (start 130.115 89.59) (end 108.115 89.59) (width 0.2) (layer "F.Cu") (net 3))
 (segment (start 105.345 92.36) (end 105.345 92.86) (width 0.2) (layer "F.Cu") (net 3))
 (segment (start 109.79 97.305) (end 109.79 102.065) (width 0.2) (layer "F.Cu") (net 3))
 (segment (start 118.615 100.59) (end 120.165 100.59) (width 0.2) (layer "F.Cu") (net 5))
 (segment (start 117.44 101.765) (end 117.615 101.59) (width 0.2) (layer "F.Cu") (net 5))
 (segment (start 115.615 101.765) (end 117.44 101.765) (width 0.2) (layer "F.Cu") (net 5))
 (segment (start 117.615 101.59) (end 118.615 100.59) (width 0.2) (layer "F.Cu") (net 5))
 (segment (start 92.465 100.565) (end 92.79 100.89) (width 0.2) (layer "F.Cu") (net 18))
 (segment (start 94.79116 103.105) (end 92.79 101.10384) (width 0.2) (layer "F.Cu") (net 18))
 (segment (start 92.79 101.10384) (end 92.79 100.89) (width 0.2) (layer "F.Cu") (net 18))
 (segment (start 95.34 103.105) (end 94.79116 103.105) (width 0.2) (layer "F.Cu") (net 18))
 (segment (start 90.79 100.565) (end 92.465 100.565) (width 0.2) (layer "F.Cu") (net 18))
 (segment (start 101.88 98.025) (end 102.84 97.065) (width 0.2) (layer "F.Cu") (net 25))
 (segment (start 100.29 98.025) (end 101.88 98.025) (width 0.2) (layer "F.Cu") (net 25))
 (segment (start 125.615 105.59) (end 125.615 103.63) (width 0.2) (layer "F.Cu") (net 12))
 (segment (start 125.615 103.63) (end 125.115 103.13) (width 0.2) (layer "F.Cu") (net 12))
 (segment (start 102.42 99.785) (end 102.115 100.09) (width 0.2) (layer "F.Cu") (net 2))
 (segment (start 103.49 99.785) (end 102.42 99.785) (width 0.2) (layer "F.Cu") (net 2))
 (via (at 102.115 100.09) (size 0.6) (drill 0.3) (layers "F.Cu" "B.Cu") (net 2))
 (via (at 100.29 99.295) (size 0.6) (drill 0.3) (layers "F.Cu" "B.Cu") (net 2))
 (segment (start 100.585 99.59) (end 101.615 99.59) (width 0.2) (layer "B.Cu") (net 2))
 (segment (start 101.615 99.59) (end 102.115 100.09) (width 0.2) (layer "B.Cu") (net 2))
 (segment (start 100.29 99.295) (end 100.585 99.59) (width 0.2) (layer "B.Cu") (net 2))
 (segment (start 127.335 98.31) (end 127.115 98.09) (width 0.2) (layer "F.Cu") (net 16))
 (segment (start 128.315 98.31) (end 127.335 98.31) (width 0.2) (layer "F.Cu") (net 16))
 (via (at 127.115 98.09) (size 0.6) (drill 0.3) (layers "F.Cu" "B.Cu") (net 16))
 (via (at 125.115 96.78) (size 0.6) (drill 0.3) (layers "F.Cu" "B.Cu") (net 16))
 (segment (start 127.115 98.09) (end 125.805 96.78) (width 0.2) (layer "B.Cu") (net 16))
 (segment (start 125.805 96.78) (end 125.115 96.78) (width 0.2) (layer "B.Cu") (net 16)))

